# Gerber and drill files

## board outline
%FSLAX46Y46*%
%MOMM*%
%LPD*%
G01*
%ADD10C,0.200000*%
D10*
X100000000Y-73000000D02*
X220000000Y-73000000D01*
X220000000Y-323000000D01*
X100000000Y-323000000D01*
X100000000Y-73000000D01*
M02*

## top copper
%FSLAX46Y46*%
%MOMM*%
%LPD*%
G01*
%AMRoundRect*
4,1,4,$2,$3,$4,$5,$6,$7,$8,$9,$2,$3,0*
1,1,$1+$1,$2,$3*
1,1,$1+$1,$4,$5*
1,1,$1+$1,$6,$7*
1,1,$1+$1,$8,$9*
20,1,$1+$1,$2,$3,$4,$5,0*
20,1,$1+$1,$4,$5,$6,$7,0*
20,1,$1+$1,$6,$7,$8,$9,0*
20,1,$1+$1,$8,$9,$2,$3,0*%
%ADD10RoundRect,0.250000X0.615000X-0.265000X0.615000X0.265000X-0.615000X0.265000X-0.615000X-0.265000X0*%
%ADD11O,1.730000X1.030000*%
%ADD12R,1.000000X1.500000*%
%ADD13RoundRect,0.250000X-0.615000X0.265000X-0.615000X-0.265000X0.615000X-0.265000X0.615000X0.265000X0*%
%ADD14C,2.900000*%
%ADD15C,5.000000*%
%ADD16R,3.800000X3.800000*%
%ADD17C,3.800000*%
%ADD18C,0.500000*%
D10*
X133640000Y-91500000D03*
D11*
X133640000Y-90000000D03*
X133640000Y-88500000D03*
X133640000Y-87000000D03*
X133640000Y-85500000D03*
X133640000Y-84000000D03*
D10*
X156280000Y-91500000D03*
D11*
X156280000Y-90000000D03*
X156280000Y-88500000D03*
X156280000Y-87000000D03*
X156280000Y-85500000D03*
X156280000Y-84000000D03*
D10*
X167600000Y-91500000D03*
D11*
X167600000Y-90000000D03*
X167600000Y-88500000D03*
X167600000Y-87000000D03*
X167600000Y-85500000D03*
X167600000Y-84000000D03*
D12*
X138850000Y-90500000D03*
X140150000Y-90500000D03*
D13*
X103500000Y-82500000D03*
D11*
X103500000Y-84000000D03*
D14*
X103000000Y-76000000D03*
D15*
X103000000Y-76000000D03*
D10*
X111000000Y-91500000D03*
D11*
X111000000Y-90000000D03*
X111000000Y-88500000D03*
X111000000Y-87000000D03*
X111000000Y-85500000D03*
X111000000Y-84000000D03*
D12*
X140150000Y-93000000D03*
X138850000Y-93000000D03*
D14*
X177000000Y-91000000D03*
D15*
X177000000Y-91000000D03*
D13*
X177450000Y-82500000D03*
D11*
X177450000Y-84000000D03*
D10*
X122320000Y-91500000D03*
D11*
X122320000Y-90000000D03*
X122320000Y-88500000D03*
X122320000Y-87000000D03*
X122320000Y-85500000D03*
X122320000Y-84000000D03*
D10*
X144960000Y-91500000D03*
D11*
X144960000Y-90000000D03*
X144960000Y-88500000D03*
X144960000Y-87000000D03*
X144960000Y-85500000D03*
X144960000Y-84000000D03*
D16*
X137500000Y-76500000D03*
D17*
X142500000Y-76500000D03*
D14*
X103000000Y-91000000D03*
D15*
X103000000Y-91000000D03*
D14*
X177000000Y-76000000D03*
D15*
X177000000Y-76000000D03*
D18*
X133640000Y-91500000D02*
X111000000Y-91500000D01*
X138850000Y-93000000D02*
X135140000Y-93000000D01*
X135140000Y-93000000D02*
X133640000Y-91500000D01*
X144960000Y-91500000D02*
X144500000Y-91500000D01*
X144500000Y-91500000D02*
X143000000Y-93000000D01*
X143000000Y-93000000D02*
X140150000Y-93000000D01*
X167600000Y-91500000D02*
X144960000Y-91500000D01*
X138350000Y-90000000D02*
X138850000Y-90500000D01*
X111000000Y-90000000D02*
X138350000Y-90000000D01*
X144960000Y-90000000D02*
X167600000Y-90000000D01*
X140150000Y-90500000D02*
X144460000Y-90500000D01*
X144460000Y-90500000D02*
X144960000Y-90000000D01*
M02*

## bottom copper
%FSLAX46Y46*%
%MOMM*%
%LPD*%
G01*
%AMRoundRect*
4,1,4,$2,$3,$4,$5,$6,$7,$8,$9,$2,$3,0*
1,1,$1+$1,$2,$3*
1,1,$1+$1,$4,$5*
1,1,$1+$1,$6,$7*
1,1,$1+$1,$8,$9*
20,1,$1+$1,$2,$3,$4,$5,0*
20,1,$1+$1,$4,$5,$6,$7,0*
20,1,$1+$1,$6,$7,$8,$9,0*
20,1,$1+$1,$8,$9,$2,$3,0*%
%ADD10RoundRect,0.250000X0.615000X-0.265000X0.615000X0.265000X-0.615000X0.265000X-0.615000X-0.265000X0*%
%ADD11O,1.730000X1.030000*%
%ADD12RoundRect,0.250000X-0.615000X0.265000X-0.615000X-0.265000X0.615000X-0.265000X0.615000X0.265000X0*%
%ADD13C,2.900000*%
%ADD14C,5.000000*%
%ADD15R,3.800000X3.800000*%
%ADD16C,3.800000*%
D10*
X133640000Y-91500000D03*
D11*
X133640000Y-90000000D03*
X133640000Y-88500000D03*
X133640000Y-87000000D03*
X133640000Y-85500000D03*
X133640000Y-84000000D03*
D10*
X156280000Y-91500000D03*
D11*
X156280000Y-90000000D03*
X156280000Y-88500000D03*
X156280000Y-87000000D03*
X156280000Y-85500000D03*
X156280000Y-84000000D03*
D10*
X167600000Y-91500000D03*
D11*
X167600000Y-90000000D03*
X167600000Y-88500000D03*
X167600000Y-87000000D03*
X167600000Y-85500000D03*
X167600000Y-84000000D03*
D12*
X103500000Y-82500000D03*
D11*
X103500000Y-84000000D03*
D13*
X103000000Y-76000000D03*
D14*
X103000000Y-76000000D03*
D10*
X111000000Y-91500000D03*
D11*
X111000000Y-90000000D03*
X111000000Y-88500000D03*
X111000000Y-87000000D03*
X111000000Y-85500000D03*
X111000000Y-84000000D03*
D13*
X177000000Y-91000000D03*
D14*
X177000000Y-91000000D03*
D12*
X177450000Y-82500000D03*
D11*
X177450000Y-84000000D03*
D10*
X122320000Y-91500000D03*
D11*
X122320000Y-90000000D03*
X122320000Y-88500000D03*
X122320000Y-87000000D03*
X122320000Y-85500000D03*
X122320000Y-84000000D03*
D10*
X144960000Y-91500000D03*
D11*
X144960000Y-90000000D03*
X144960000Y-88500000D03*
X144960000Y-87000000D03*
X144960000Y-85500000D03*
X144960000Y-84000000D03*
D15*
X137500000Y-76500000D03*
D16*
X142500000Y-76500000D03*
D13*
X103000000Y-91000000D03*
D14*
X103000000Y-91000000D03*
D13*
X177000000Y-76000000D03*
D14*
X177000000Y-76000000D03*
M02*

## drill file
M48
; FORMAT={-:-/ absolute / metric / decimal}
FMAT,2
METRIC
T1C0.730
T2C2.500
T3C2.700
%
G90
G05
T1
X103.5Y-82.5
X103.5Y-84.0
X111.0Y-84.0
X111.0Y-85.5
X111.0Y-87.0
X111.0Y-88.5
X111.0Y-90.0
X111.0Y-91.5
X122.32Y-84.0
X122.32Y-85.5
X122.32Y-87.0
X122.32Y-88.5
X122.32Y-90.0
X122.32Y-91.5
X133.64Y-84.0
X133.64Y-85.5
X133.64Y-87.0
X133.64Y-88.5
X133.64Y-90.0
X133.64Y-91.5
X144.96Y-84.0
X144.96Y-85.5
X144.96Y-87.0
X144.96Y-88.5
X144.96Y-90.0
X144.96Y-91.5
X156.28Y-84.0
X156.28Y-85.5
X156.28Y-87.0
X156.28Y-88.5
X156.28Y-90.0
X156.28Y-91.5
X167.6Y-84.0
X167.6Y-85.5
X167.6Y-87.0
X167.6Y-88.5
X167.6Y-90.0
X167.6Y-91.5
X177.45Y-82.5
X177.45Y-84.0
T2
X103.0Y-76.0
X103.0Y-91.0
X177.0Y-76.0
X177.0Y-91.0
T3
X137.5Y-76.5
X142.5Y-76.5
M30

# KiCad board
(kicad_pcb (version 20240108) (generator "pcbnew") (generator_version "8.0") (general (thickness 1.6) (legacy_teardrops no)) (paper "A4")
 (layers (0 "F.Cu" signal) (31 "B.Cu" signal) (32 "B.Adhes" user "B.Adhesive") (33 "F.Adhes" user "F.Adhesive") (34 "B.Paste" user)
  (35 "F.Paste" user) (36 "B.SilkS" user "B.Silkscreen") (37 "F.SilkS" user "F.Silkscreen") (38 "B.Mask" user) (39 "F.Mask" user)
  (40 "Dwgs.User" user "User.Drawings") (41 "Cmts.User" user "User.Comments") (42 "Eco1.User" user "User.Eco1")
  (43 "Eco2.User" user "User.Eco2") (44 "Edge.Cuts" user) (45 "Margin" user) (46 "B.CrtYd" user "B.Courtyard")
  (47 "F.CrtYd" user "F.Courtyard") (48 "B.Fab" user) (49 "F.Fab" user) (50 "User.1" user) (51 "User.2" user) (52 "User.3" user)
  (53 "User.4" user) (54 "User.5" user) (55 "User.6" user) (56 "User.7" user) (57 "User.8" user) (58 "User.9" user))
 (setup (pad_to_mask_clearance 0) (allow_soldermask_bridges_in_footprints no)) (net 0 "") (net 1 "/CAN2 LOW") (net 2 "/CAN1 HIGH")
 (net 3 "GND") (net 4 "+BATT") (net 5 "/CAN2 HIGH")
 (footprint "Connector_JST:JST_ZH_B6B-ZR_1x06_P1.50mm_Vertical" (layer "F.Cu") (at 133.64 91.5 90)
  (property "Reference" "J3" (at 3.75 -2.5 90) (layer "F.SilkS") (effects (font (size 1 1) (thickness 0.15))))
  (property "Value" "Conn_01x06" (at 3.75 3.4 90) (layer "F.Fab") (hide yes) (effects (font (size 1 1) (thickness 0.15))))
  (pad "1" thru_hole roundrect (at 0 0 90) (size 1.03 1.73) (drill 0.73) (layers "*.Cu" "*.Mask") (remove_unused_layers no)
   (roundrect_rratio 0.242718) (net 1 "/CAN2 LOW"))
  (pad "2" thru_hole oval (at 1.5 0 90) (size 1.03 1.73) (drill 0.73) (layers "*.Cu" "*.Mask") (remove_unused_layers no)
   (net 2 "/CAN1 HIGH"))
  (pad "3" thru_hole oval (at 3 0 90) (size 1.03 1.73) (drill 0.73) (layers "*.Cu" "*.Mask") (remove_unused_layers no) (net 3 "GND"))
  (pad "4" thru_hole oval (at 4.5 0 90) (size 1.03 1.73) (drill 0.73) (layers "*.Cu" "*.Mask") (remove_unused_layers no) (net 3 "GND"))
  (pad "5" thru_hole oval (at 6 0 90) (size 1.03 1.73) (drill 0.73) (layers "*.Cu" "*.Mask") (remove_unused_layers no) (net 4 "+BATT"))
  (pad "6" thru_hole oval (at 7.5 0 90) (size 1.03 1.73) (drill 0.73) (layers "*.Cu" "*.Mask") (remove_unused_layers no) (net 4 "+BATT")))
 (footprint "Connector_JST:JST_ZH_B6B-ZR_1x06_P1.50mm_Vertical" (layer "F.Cu") (at 156.28 91.5 90)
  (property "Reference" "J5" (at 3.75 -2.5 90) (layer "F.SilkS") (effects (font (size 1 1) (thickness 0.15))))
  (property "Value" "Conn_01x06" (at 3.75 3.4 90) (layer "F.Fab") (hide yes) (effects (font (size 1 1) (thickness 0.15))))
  (pad "1" thru_hole roundrect (at 0 0 90) (size 1.03 1.73) (drill 0.73) (layers "*.Cu" "*.Mask") (remove_unused_layers no)
   (roundrect_rratio 0.242718) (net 1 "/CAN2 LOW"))
  (pad "2" thru_hole oval (at 1.5 0 90) (size 1.03 1.73) (drill 0.73) (layers "*.Cu" "*.Mask") (remove_unused_layers no)
   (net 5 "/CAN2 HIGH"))
  (pad "3" thru_hole oval (at 3 0 90) (size 1.03 1.73) (drill 0.73) (layers "*.Cu" "*.Mask") (remove_unused_layers no) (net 3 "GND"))
  (pad "4" thru_hole oval (at 4.5 0 90) (size 1.03 1.73) (drill 0.73) (layers "*.Cu" "*.Mask") (remove_unused_layers no) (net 3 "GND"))
  (pad "5" thru_hole oval (at 6 0 90) (size 1.03 1.73) (drill 0.73) (layers "*.Cu" "*.Mask") (remove_unused_layers no) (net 4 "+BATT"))
  (pad "6" thru_hole oval (at 7.5 0 90) (size 1.03 1.73) (drill 0.73) (layers "*.Cu" "*.Mask") (remove_unused_layers no) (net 4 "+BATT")))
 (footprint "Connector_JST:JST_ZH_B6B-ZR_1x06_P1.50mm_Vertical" (layer "F.Cu") (at 167.6 91.5 90)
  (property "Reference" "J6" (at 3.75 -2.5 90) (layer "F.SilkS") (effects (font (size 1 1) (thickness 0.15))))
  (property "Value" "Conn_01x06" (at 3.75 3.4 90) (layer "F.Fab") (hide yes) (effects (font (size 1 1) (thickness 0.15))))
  (pad "1" thru_hole roundrect (at 0 0 90) (size 1.03 1.73) (drill 0.73) (layers "*.Cu" "*.Mask") (remove_unused_layers no)
   (roundrect_rratio 0.242718) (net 1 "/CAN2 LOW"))
  (pad "2" thru_hole oval (at 1.5 0 90) (size 1.03 1.73) (drill 0.73) (layers "*.Cu" "*.Mask") (remove_unused_layers no)
   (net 5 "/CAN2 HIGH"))
  (pad "3" thru_hole oval (at 3 0 90) (size 1.03 1.73) (drill 0.73) (layers "*.Cu" "*.Mask") (remove_unused_layers no) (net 3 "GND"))
  (pad "4" thru_hole oval (at 4.5 0 90) (size 1.03 1.73) (drill 0.73) (layers "*.Cu" "*.Mask") (remove_unused_layers no) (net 3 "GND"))
  (pad "5" thru_hole oval (at 6 0 90) (size 1.03 1.73) (drill 0.73) (layers "*.Cu" "*.Mask") (remove_unused_layers no) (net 4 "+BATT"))
  (pad "6" thru_hole oval (at 7.5 0 90) (size 1.03 1.73) (drill 0.73) (layers "*.Cu" "*.Mask") (remove_unused_layers no) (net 4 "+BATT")))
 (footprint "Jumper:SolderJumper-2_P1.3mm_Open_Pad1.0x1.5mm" (layer "F.Cu") (at 139.5 90.5)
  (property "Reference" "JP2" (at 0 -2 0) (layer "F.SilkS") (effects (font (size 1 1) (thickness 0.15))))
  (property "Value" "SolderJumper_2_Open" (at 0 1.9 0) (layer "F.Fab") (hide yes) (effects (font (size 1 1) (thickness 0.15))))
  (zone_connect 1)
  (pad "1" smd rect (at -0.65 0) (size 1 1.5) (layers "F.Cu" "F.Mask") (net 2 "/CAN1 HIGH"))
  (pad "2" smd rect (at 0.65 0) (size 1 1.5) (layers "F.Cu" "F.Mask") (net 5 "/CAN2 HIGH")))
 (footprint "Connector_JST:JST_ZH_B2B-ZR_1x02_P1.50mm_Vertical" (layer "F.Cu") (at 103.5 82.5 -90)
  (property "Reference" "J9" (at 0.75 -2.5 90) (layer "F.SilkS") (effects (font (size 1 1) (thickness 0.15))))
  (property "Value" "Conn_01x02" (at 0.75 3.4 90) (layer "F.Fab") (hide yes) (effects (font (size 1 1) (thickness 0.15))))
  (pad "1" thru_hole roundrect (at 0 0 270) (size 1.03 1.73) (drill 0.73) (layers "*.Cu" "*.Mask") (remove_unused_layers no)
   (roundrect_rratio 0.242718) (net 2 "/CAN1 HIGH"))
  (pad "2" thru_hole oval (at 1.5 0 270) (size 1.03 1.73) (drill 0.73) (layers "*.Cu" "*.Mask") (remove_unused_layers no)
   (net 1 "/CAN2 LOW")))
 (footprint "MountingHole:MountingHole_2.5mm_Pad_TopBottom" (layer "F.Cu") (at 103 76)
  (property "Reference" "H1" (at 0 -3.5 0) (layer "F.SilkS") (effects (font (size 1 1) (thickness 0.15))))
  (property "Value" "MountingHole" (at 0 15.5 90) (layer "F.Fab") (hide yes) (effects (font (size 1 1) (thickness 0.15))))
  (pad "1" thru_hole circle (at 0 0) (size 2.9 2.9) (drill 2.5) (layers "*.Cu" "*.Mask") (remove_unused_layers no))
  (pad "1" connect circle (at 0 0) (size 5 5) (layers "F.Cu" "F.Mask"))
  (pad "1" connect circle (at 0 0) (size 5 5) (layers "B.Cu" "B.Mask")))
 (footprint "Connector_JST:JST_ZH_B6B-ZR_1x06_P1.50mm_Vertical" (layer "F.Cu") (at 111 91.5 90)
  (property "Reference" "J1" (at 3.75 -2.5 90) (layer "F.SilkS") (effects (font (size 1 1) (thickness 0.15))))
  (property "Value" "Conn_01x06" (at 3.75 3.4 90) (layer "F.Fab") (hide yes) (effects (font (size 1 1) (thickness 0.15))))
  (pad "1" thru_hole roundrect (at 0 0 90) (size 1.03 1.73) (drill 0.73) (layers "*.Cu" "*.Mask") (remove_unused_layers no)
   (roundrect_rratio 0.242718) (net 1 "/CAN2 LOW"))
  (pad "2" thru_hole oval (at 1.5 0 90) (size 1.03 1.73) (drill 0.73) (layers "*.Cu" "*.Mask") (remove_unused_layers no)
   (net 2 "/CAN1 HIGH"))
  (pad "3" thru_hole oval (at 3 0 90) (size 1.03 1.73) (drill 0.73) (layers "*.Cu" "*.Mask") (remove_unused_layers no) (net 3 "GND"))
  (pad "4" thru_hole oval (at 4.5 0 90) (size 1.03 1.73) (drill 0.73) (layers "*.Cu" "*.Mask") (remove_unused_layers no) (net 3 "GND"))
  (pad "5" thru_hole oval (at 6 0 90) (size 1.03 1.73) (drill 0.73) (layers "*.Cu" "*.Mask") (remove_unused_layers no) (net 4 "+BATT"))
  (pad "6" thru_hole oval (at 7.5 0 90) (size 1.03 1.73) (drill 0.73) (layers "*.Cu" "*.Mask") (remove_unused_layers no) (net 4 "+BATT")))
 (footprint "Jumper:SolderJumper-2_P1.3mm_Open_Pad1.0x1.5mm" (layer "F.Cu") (at 139.5 93 180)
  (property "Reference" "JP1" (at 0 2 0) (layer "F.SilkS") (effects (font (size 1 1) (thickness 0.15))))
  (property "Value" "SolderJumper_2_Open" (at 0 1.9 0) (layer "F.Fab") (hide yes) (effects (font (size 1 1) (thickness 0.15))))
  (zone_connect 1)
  (pad "1" smd rect (at -0.65 0 180) (size 1 1.5) (layers "F.Cu" "F.Mask") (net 1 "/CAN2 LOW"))
  (pad "2" smd rect (at 0.65 0 180) (size 1 1.5) (layers "F.Cu" "F.Mask") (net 1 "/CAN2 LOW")))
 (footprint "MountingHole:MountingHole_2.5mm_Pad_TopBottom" (layer "F.Cu") (at 177 91)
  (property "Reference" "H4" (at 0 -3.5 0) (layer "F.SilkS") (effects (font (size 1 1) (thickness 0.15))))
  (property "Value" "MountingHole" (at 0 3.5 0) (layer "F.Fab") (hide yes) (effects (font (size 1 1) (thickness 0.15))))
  (pad "1" thru_hole circle (at 0 0) (size 2.9 2.9) (drill 2.5) (layers "*.Cu" "*.Mask") (remove_unused_layers no))
  (pad "1" connect circle (at 0 0) (size 5 5) (layers "F.Cu" "F.Mask"))
  (pad "1" connect circle (at 0 0) (size 5 5) (layers "B.Cu" "B.Mask")))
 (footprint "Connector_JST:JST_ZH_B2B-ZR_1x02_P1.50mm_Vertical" (layer "F.Cu") (at 177.45 82.5 -90)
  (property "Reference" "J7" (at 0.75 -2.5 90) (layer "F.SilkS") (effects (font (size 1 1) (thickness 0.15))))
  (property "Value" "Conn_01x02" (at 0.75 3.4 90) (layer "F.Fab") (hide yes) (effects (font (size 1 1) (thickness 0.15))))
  (pad "1" thru_hole roundrect (at 0 0 270) (size 1.03 1.73) (drill 0.73) (layers "*.Cu" "*.Mask") (remove_unused_layers no)
   (roundrect_rratio 0.242718) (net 5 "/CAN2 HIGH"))
  (pad "2" thru_hole oval (at 1.5 0 270) (size 1.03 1.73) (drill 0.73) (layers "*.Cu" "*.Mask") (remove_unused_layers no)
   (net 1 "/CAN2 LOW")))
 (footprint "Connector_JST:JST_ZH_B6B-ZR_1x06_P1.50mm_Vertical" (layer "F.Cu") (at 122.32 91.5 90)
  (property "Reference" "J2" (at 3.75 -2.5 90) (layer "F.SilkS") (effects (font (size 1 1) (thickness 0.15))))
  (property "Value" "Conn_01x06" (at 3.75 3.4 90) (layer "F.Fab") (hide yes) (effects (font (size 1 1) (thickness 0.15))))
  (pad "1" thru_hole roundrect (at 0 0 90) (size 1.03 1.73) (drill 0.73) (layers "*.Cu" "*.Mask") (remove_unused_layers no)
   (roundrect_rratio 0.242718) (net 1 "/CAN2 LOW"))
  (pad "2" thru_hole oval (at 1.5 0 90) (size 1.03 1.73) (drill 0.73) (layers "*.Cu" "*.Mask") (remove_unused_layers no)
   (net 2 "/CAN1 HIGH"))
  (pad "3" thru_hole oval (at 3 0 90) (size 1.03 1.73) (drill 0.73) (layers "*.Cu" "*.Mask") (remove_unused_layers no) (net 3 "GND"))
  (pad "4" thru_hole oval (at 4.5 0 90) (size 1.03 1.73) (drill 0.73) (layers "*.Cu" "*.Mask") (remove_unused_layers no) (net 3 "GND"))
  (pad "5" thru_hole oval (at 6 0 90) (size 1.03 1.73) (drill 0.73) (layers "*.Cu" "*.Mask") (remove_unused_layers no) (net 4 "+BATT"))
  (pad "6" thru_hole oval (at 7.5 0 90) (size 1.03 1.73) (drill 0.73) (layers "*.Cu" "*.Mask") (remove_unused_layers no) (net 4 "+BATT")))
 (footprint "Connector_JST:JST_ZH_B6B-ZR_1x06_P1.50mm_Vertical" (layer "F.Cu") (at 144.96 91.5 90)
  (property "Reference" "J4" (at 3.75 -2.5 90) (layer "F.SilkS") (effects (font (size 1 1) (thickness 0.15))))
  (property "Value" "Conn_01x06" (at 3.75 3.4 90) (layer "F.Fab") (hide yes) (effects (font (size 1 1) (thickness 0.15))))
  (pad "1" thru_hole roundrect (at 0 0 90) (size 1.03 1.73) (drill 0.73) (layers "*.Cu" "*.Mask") (remove_unused_layers no)
   (roundrect_rratio 0.242718) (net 1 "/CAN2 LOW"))
  (pad "2" thru_hole oval (at 1.5 0 90) (size 1.03 1.73) (drill 0.73) (layers "*.Cu" "*.Mask") (remove_unused_layers no)
   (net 5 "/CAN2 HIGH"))
  (pad "3" thru_hole oval (at 3 0 90) (size 1.03 1.73) (drill 0.73) (layers "*.Cu" "*.Mask") (remove_unused_layers no) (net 3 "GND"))
  (pad "4" thru_hole oval (at 4.5 0 90) (size 1.03 1.73) (drill 0.73) (layers "*.Cu" "*.Mask") (remove_unused_layers no) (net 3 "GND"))
  (pad "5" thru_hole oval (at 6 0 90) (size 1.03 1.73) (drill 0.73) (layers "*.Cu" "*.Mask") (remove_unused_layers no) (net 4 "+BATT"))
  (pad "6" thru_hole oval (at 7.5 0 90) (size 1.03 1.73) (drill 0.73) (layers "*.Cu" "*.Mask") (remove_unused_layers no) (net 4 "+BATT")))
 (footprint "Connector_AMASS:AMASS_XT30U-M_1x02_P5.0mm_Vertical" (layer "F.Cu") (at 137.5 76.5)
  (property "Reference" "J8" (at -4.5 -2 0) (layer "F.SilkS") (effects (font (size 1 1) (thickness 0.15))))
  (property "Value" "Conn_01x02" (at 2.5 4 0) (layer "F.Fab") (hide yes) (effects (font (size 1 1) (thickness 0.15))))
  (pad "1" thru_hole rect (at 0 0) (size 3.8 3.8) (drill 2.7) (layers "*.Cu" "*.Mask") (remove_unused_layers no) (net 3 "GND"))
  (pad "2" thru_hole circle (at 5 0) (size 3.8 3.8) (drill 2.7) (layers "*.Cu" "*.Mask") (remove_unused_layers no) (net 4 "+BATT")))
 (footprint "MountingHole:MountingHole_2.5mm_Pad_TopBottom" (layer "F.Cu") (at 103 91)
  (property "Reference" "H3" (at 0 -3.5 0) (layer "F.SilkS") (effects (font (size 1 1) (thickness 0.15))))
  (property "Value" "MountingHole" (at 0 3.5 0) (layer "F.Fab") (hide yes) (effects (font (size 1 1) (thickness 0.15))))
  (pad "1" thru_hole circle (at 0 0) (size 2.9 2.9) (drill 2.5) (layers "*.Cu" "*.Mask") (remove_unused_layers no))
  (pad "1" connect circle (at 0 0) (size 5 5) (layers "F.Cu" "F.Mask"))
  (pad "1" connect circle (at 0 0) (size 5 5) (layers "B.Cu" "B.Mask")))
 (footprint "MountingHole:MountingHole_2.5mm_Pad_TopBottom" (layer "F.Cu") (at 177 76)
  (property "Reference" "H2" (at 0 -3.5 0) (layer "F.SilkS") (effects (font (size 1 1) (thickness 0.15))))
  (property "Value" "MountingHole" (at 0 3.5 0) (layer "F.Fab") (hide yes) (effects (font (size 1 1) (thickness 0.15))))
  (pad "1" thru_hole circle (at 0 0) (size 2.9 2.9) (drill 2.5) (layers "*.Cu" "*.Mask") (remove_unused_layers no))
  (pad "1" connect circle (at 0 0) (size 5 5) (layers "F.Cu" "F.Mask"))
  (pad "1" connect circle (at 0 0) (size 5 5) (layers "B.Cu" "B.Mask")))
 (gr_rect (start 100 73) (end 220 323) (stroke (width 0.2) (type default)) (fill none) (layer "Edge.Cuts"))
 (segment (start 133.64 91.5) (end 111 91.5) (width 0.5) (layer "F.Cu") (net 1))
 (segment (start 138.85 93) (end 135.14 93) (width 0.5) (layer "F.Cu") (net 1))
 (segment (start 135.14 93) (end 133.64 91.5) (width 0.5) (layer "F.Cu") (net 1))
 (segment (start 144.96 91.5) (end 144.5 91.5) (width 0.5) (layer "F.Cu") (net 1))
 (segment (start 144.5 91.5) (end 143 93) (width 0.5) (layer "F.Cu") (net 1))
 (segment (start 143 93) (end 140.15 93) (width 0.5) (layer "F.Cu") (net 1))
 (segment (start 167.6 91.5) (end 144.96 91.5) (width 0.5) (layer "F.Cu") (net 1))
 (segment (start 138.35 90) (end 138.85 90.5) (width 0.5) (layer "F.Cu") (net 2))
 (segment (start 111 90) (end 138.35 90) (width 0.5) (layer "F.Cu") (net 2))
 (segment (start 144.96 90) (end 167.6 90) (width 0.5) (layer "F.Cu") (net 5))
 (segment (start 140.15 90.5) (end 144.46 90.5) (width 0.5) (layer "F.Cu") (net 5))
 (segment (start 144.46 90.5) (end 144.96 90) (width 0.5) (layer "F.Cu") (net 5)))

